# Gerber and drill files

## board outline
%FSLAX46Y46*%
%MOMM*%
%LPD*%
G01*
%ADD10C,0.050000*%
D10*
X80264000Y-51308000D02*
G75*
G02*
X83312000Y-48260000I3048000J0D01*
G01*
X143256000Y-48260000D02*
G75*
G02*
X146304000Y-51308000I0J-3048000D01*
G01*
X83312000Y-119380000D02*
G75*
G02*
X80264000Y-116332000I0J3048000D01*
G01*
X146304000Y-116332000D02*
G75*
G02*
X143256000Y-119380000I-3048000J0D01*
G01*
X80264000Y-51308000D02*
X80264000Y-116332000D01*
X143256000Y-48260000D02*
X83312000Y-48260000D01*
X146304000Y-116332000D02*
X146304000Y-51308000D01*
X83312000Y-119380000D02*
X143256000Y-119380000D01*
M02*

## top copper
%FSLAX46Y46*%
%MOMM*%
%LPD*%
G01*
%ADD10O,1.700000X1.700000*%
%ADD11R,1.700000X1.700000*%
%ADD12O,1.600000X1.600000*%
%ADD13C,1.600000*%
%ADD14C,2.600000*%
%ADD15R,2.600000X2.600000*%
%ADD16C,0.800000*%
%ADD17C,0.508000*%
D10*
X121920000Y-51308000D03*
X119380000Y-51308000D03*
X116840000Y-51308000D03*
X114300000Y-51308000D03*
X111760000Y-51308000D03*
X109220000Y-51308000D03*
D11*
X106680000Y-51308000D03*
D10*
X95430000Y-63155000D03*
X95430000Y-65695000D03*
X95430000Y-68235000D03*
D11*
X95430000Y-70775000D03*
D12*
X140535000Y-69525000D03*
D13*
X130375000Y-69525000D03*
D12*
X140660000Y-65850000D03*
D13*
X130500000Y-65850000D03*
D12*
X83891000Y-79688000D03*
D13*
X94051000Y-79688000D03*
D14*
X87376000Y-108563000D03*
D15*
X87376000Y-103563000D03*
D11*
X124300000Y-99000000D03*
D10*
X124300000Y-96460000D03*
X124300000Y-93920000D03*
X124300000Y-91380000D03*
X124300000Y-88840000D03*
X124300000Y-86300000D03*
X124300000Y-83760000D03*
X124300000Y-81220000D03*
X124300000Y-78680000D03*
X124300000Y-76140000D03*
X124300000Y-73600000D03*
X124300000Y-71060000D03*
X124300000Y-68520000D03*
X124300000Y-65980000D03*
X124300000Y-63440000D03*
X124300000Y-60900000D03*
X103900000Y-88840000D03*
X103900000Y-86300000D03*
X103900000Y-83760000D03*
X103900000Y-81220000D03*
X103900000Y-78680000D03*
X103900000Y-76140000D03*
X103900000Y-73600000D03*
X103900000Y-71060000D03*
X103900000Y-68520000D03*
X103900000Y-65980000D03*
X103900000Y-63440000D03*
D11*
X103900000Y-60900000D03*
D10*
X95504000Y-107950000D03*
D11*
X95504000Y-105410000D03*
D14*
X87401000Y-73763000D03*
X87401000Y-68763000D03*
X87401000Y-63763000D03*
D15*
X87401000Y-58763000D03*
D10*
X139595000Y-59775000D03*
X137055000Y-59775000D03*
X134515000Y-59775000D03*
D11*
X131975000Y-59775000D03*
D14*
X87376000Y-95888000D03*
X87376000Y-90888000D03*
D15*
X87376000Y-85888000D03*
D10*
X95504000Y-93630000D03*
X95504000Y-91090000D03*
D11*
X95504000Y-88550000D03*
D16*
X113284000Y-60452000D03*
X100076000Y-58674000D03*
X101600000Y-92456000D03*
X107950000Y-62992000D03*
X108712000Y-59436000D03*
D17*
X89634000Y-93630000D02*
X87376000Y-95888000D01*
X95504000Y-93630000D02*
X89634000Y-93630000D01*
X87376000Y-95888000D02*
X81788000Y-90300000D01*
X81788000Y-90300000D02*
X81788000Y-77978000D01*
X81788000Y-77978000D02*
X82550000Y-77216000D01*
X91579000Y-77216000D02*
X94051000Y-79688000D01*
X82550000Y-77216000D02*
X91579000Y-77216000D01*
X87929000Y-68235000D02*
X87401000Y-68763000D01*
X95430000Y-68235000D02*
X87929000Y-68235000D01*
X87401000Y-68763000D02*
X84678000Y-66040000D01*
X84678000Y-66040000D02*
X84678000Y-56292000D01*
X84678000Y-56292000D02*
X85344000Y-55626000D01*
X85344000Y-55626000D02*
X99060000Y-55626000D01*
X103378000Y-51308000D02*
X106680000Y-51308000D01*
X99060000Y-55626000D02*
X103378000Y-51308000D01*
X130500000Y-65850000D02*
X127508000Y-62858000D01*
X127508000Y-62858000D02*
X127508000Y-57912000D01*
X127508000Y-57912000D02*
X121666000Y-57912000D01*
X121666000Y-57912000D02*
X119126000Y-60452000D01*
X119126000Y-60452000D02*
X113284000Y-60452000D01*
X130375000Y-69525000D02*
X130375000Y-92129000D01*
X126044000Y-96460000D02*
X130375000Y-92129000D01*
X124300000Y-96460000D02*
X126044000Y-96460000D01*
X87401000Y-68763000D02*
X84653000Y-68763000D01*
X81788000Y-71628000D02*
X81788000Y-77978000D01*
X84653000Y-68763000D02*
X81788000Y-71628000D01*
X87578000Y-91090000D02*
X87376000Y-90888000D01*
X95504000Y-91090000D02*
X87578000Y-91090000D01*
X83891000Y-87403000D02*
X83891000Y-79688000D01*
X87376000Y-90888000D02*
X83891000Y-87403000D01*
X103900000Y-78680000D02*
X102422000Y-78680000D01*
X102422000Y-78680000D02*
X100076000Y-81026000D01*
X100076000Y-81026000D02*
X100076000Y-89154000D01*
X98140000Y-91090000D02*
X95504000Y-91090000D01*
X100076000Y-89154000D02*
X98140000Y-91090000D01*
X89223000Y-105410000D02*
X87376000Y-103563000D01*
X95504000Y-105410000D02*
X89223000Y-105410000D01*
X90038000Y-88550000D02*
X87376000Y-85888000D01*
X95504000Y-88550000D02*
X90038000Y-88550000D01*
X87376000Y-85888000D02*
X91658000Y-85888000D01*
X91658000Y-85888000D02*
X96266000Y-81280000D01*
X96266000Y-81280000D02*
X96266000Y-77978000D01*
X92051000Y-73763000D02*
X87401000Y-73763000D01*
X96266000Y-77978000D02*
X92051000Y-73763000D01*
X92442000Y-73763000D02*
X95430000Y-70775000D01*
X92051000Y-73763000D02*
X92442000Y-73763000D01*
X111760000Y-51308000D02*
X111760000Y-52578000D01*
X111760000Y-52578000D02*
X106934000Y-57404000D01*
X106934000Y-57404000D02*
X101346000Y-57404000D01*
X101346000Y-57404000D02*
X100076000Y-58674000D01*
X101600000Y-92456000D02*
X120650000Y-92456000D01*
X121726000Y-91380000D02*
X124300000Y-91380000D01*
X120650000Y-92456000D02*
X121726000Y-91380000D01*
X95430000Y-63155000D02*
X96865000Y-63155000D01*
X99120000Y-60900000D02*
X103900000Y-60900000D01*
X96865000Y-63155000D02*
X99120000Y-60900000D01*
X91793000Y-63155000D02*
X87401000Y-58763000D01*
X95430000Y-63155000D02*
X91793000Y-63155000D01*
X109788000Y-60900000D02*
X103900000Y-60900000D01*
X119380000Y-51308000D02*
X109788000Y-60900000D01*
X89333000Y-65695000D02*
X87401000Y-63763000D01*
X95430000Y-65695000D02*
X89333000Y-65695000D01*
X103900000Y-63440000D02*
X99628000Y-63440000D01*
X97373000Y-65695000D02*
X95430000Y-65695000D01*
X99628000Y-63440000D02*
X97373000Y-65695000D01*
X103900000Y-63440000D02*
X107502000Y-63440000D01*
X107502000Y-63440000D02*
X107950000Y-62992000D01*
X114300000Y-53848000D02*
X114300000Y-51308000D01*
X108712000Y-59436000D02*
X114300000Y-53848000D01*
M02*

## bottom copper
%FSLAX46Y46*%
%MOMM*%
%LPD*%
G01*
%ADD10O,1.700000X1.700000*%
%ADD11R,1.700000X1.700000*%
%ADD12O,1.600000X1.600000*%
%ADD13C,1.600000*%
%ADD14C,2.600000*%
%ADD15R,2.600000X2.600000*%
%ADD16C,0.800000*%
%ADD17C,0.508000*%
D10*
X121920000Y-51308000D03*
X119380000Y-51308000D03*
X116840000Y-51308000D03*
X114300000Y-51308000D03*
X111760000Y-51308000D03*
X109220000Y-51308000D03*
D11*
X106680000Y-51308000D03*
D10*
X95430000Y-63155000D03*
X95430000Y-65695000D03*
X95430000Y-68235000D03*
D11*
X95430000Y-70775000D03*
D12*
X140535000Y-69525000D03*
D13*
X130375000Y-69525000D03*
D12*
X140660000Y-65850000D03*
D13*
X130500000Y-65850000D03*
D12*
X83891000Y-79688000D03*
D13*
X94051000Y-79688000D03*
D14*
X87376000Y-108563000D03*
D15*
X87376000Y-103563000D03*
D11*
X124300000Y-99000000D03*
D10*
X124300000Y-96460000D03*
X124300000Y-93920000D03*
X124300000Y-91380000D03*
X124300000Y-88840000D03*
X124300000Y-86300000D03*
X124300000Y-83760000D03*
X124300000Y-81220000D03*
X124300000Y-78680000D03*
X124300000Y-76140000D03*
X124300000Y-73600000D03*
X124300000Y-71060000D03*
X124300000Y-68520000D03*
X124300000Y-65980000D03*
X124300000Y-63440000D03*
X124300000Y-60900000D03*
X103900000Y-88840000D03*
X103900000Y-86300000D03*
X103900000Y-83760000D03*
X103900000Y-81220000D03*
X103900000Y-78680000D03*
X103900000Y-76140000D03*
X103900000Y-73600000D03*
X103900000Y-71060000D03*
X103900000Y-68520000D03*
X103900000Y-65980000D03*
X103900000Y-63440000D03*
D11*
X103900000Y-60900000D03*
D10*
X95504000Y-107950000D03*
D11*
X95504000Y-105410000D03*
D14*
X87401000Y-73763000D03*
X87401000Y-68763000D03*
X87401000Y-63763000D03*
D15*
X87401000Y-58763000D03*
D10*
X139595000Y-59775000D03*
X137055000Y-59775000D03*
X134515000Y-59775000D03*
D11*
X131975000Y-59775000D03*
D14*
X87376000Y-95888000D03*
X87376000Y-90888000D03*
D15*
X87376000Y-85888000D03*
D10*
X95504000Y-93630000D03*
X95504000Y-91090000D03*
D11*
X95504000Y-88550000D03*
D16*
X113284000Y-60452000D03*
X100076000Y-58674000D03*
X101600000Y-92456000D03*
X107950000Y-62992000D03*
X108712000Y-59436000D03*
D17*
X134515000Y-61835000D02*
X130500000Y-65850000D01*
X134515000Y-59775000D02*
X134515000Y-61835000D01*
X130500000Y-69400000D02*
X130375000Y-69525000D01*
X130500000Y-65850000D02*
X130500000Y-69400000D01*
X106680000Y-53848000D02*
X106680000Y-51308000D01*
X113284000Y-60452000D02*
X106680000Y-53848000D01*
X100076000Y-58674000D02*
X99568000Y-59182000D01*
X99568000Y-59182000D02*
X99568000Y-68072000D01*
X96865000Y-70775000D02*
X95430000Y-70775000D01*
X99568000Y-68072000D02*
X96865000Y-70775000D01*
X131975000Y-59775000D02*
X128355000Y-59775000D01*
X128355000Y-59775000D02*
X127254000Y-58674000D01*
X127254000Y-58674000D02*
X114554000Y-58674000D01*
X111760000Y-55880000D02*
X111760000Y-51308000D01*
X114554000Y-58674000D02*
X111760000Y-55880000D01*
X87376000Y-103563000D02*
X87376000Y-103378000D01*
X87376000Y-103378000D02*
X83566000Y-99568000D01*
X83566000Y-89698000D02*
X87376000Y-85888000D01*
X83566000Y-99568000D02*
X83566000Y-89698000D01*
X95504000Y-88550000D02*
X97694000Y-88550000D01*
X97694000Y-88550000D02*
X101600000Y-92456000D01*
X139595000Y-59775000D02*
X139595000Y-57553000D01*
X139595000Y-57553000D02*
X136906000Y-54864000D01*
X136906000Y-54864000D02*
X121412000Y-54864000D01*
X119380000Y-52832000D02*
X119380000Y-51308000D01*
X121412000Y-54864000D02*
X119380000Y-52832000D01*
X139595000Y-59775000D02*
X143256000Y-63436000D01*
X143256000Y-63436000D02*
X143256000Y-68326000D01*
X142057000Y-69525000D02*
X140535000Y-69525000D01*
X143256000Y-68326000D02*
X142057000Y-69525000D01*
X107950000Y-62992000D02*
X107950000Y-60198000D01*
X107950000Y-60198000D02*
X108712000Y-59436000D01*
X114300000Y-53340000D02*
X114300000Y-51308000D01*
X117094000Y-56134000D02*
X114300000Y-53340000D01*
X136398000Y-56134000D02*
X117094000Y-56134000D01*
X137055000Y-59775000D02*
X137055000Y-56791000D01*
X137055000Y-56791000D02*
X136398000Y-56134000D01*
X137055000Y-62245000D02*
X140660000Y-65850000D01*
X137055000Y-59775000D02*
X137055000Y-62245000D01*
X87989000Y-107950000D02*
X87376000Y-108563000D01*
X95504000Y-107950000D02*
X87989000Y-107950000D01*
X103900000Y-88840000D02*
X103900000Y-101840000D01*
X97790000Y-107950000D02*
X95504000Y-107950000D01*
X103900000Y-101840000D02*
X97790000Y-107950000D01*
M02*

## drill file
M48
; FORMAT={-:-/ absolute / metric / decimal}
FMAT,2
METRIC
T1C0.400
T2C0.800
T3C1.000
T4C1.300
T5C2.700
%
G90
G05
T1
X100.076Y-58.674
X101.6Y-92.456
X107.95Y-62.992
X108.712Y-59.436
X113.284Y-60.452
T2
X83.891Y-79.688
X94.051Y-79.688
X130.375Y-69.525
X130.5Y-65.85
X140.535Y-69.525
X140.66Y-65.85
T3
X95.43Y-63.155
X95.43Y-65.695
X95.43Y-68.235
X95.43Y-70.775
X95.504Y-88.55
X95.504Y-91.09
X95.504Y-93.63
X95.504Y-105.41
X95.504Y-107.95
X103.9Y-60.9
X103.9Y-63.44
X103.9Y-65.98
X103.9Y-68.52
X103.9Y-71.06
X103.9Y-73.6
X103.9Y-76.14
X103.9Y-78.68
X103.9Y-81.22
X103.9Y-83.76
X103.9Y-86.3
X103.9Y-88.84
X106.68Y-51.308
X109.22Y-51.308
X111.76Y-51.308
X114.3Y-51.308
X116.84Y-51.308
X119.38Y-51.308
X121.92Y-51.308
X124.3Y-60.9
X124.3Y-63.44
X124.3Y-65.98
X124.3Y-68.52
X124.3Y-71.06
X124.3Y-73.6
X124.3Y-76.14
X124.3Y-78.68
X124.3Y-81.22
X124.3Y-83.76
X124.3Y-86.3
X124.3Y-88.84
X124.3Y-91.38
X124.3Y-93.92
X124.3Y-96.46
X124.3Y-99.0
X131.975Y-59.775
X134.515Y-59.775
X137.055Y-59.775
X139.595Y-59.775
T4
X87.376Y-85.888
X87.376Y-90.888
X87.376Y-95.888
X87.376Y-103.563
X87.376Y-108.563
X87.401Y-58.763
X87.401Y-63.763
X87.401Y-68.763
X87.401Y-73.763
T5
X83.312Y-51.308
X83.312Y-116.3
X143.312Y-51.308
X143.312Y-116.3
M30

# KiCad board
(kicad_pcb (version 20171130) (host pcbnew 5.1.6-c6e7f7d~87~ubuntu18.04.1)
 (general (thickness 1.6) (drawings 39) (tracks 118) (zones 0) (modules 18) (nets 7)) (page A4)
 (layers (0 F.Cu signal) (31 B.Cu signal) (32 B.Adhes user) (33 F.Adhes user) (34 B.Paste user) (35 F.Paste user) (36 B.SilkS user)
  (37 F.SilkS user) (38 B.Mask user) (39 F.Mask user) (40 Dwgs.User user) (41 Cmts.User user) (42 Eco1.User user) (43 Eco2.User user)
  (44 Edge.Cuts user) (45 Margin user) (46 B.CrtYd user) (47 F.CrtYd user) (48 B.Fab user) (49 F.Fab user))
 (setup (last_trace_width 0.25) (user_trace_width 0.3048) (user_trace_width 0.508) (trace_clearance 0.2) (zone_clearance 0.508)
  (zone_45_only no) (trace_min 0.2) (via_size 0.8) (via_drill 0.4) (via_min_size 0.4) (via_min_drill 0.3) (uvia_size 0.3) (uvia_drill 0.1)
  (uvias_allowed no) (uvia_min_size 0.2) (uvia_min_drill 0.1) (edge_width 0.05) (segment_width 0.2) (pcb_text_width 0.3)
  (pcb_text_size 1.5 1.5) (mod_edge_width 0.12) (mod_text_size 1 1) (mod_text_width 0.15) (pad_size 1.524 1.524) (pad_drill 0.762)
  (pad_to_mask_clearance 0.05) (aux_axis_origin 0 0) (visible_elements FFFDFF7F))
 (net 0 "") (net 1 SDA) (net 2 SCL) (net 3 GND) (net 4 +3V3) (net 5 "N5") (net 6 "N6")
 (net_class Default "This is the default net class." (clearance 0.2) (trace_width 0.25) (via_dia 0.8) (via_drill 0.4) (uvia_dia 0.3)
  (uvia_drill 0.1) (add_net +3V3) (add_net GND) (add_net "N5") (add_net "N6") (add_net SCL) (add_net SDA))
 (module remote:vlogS (layer F.Cu) (at 136.652 107.442)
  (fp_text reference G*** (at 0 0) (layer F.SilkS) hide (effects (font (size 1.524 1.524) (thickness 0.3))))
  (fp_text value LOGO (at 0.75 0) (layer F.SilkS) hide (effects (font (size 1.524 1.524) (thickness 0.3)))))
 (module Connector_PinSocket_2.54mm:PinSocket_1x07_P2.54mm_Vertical (layer F.Cu) (at 106.68 51.308 90)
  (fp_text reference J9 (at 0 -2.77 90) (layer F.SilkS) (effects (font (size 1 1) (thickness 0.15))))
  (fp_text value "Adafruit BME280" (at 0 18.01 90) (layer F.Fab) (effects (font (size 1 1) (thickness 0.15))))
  (pad 7 thru_hole oval (at 0 15.24 90) (size 1.7 1.7) (drill 1) (layers *.Cu *.Mask))
  (pad 6 thru_hole oval (at 0 12.7 90) (size 1.7 1.7) (drill 1) (layers *.Cu *.Mask) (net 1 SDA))
  (pad 5 thru_hole oval (at 0 10.16 90) (size 1.7 1.7) (drill 1) (layers *.Cu *.Mask))
  (pad 4 thru_hole oval (at 0 7.62 90) (size 1.7 1.7) (drill 1) (layers *.Cu *.Mask) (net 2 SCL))
  (pad 3 thru_hole oval (at 0 5.08 90) (size 1.7 1.7) (drill 1) (layers *.Cu *.Mask) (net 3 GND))
  (pad 2 thru_hole oval (at 0 2.54 90) (size 1.7 1.7) (drill 1) (layers *.Cu *.Mask))
  (pad 1 thru_hole rect (at 0 0 90) (size 1.7 1.7) (drill 1) (layers *.Cu *.Mask) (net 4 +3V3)))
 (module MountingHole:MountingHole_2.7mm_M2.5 (layer F.Cu) (at 143.312 116.3)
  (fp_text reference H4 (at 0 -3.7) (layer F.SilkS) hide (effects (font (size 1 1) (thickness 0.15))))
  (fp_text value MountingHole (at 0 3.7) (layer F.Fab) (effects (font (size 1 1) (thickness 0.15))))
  (pad 1 np_thru_hole circle (at 0 0) (size 2.7 2.7) (drill 2.7) (layers *.Cu *.Mask)))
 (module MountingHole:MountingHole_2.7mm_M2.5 (layer F.Cu) (at 83.312 116.3)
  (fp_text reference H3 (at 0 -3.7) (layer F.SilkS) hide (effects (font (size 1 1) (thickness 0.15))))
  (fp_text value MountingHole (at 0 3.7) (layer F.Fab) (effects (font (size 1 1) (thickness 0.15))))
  (pad 1 np_thru_hole circle (at 0 0) (size 2.7 2.7) (drill 2.7) (layers *.Cu *.Mask)))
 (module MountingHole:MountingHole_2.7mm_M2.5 (layer F.Cu) (at 143.312 51.308)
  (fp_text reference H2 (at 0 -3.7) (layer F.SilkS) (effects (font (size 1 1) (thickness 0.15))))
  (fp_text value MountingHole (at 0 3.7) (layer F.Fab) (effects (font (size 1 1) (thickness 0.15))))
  (pad 1 np_thru_hole circle (at 0 0) (size 2.7 2.7) (drill 2.7) (layers *.Cu *.Mask)))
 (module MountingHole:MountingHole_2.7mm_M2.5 (layer F.Cu) (at 83.312 51.308)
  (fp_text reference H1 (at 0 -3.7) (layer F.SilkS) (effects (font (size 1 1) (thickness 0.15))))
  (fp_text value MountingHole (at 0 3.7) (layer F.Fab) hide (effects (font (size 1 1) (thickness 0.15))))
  (pad 1 np_thru_hole circle (at 0 0) (size 2.7 2.7) (drill 2.7) (layers *.Cu *.Mask)))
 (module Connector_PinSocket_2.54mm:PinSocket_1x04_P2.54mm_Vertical (layer F.Cu) (at 95.43 70.775 180)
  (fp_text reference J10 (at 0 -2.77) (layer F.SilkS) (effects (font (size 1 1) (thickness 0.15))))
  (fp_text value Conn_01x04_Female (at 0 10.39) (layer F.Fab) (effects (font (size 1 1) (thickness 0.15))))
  (pad 4 thru_hole oval (at 0 7.62 180) (size 1.7 1.7) (drill 1) (layers *.Cu *.Mask) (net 1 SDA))
  (pad 3 thru_hole oval (at 0 5.08 180) (size 1.7 1.7) (drill 1) (layers *.Cu *.Mask) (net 2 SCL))
  (pad 2 thru_hole oval (at 0 2.54 180) (size 1.7 1.7) (drill 1) (layers *.Cu *.Mask) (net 4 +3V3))
  (pad 1 thru_hole rect (at 0 0 180) (size 1.7 1.7) (drill 1) (layers *.Cu *.Mask) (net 3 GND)))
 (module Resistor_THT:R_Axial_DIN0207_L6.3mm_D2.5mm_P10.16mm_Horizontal (layer F.Cu) (at 130.375 69.525)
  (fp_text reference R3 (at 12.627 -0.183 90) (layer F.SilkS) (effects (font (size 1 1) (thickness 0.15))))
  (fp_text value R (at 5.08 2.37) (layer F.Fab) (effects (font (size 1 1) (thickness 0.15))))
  (pad 2 thru_hole oval (at 10.16 0) (size 1.6 1.6) (drill 0.8) (layers *.Cu *.Mask) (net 1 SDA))
  (pad 1 thru_hole circle (at 0 0) (size 1.6 1.6) (drill 0.8) (layers *.Cu *.Mask) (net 4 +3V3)))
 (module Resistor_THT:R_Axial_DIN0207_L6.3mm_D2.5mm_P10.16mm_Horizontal (layer F.Cu) (at 130.5 65.85)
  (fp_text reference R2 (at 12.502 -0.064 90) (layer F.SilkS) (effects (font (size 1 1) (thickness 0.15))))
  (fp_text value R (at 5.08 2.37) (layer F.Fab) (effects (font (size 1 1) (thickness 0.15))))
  (pad 2 thru_hole oval (at 10.16 0) (size 1.6 1.6) (drill 0.8) (layers *.Cu *.Mask) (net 2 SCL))
  (pad 1 thru_hole circle (at 0 0) (size 1.6 1.6) (drill 0.8) (layers *.Cu *.Mask) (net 4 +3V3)))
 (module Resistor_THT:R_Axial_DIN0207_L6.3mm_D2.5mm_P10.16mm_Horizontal (layer F.Cu) (at 94.051 79.688 180)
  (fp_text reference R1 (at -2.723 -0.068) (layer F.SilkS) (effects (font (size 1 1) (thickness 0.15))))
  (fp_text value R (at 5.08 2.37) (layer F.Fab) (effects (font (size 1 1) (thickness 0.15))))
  (pad 2 thru_hole oval (at 10.16 0 180) (size 1.6 1.6) (drill 0.8) (layers *.Cu *.Mask) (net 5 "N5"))
  (pad 1 thru_hole circle (at 0 0 180) (size 1.6 1.6) (drill 0.8) (layers *.Cu *.Mask) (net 4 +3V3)))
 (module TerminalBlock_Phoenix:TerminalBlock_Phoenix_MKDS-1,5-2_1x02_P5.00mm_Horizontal (layer F.Cu) (at 87.376 103.563 270)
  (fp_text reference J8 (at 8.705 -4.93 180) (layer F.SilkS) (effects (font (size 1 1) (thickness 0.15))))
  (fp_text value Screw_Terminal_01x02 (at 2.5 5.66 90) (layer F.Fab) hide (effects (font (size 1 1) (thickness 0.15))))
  (pad 2 thru_hole circle (at 5 0 270) (size 2.6 2.6) (drill 1.3) (layers *.Cu *.Mask) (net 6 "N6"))
  (pad 1 thru_hole rect (at 0 0 270) (size 2.6 2.6) (drill 1.3) (layers *.Cu *.Mask) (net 3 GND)))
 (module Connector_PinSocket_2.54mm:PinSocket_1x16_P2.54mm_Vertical (layer F.Cu) (at 124.3 99 180)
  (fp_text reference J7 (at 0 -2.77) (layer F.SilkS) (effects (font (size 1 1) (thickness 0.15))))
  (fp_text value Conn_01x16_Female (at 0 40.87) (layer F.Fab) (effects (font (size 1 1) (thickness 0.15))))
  (pad 1 thru_hole rect (at 0 0 180) (size 1.7 1.7) (drill 1) (layers *.Cu *.Mask))
  (pad 2 thru_hole oval (at 0 2.54 180) (size 1.7 1.7) (drill 1) (layers *.Cu *.Mask) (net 4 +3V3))
  (pad 3 thru_hole oval (at 0 5.08 180) (size 1.7 1.7) (drill 1) (layers *.Cu *.Mask))
  (pad 4 thru_hole oval (at 0 7.62 180) (size 1.7 1.7) (drill 1) (layers *.Cu *.Mask) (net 3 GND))
  (pad 5 thru_hole oval (at 0 10.16 180) (size 1.7 1.7) (drill 1) (layers *.Cu *.Mask))
  (pad 6 thru_hole oval (at 0 12.7 180) (size 1.7 1.7) (drill 1) (layers *.Cu *.Mask))
  (pad 7 thru_hole oval (at 0 15.24 180) (size 1.7 1.7) (drill 1) (layers *.Cu *.Mask))
  (pad 8 thru_hole oval (at 0 17.78 180) (size 1.7 1.7) (drill 1) (layers *.Cu *.Mask))
  (pad 9 thru_hole oval (at 0 20.32 180) (size 1.7 1.7) (drill 1) (layers *.Cu *.Mask))
  (pad 10 thru_hole oval (at 0 22.86 180) (size 1.7 1.7) (drill 1) (layers *.Cu *.Mask))
  (pad 11 thru_hole oval (at 0 25.4 180) (size 1.7 1.7) (drill 1) (layers *.Cu *.Mask))
  (pad 12 thru_hole oval (at 0 27.94 180) (size 1.7 1.7) (drill 1) (layers *.Cu *.Mask))
  (pad 13 thru_hole oval (at 0 30.48 180) (size 1.7 1.7) (drill 1) (layers *.Cu *.Mask))
  (pad 14 thru_hole oval (at 0 33.02 180) (size 1.7 1.7) (drill 1) (layers *.Cu *.Mask))
  (pad 15 thru_hole oval (at 0 35.56 180) (size 1.7 1.7) (drill 1) (layers *.Cu *.Mask))
  (pad 16 thru_hole oval (at 0 38.1 180) (size 1.7 1.7) (drill 1) (layers *.Cu *.Mask)))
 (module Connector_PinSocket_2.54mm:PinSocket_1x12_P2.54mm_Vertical (layer F.Cu) (at 103.9 60.9)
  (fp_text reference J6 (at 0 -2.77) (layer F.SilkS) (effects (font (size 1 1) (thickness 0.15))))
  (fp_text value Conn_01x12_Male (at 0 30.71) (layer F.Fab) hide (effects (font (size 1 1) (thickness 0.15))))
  (pad 12 thru_hole oval (at 0 27.94) (size 1.7 1.7) (drill 1) (layers *.Cu *.Mask) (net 6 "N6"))
  (pad 11 thru_hole oval (at 0 25.4) (size 1.7 1.7) (drill 1) (layers *.Cu *.Mask))
  (pad 10 thru_hole oval (at 0 22.86) (size 1.7 1.7) (drill 1) (layers *.Cu *.Mask))
  (pad 9 thru_hole oval (at 0 20.32) (size 1.7 1.7) (drill 1) (layers *.Cu *.Mask))
  (pad 8 thru_hole oval (at 0 17.78) (size 1.7 1.7) (drill 1) (layers *.Cu *.Mask) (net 5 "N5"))
  (pad 7 thru_hole oval (at 0 15.24) (size 1.7 1.7) (drill 1) (layers *.Cu *.Mask))
  (pad 6 thru_hole oval (at 0 12.7) (size 1.7 1.7) (drill 1) (layers *.Cu *.Mask))
  (pad 5 thru_hole oval (at 0 10.16) (size 1.7 1.7) (drill 1) (layers *.Cu *.Mask))
  (pad 4 thru_hole oval (at 0 7.62) (size 1.7 1.7) (drill 1) (layers *.Cu *.Mask))
  (pad 3 thru_hole oval (at 0 5.08) (size 1.7 1.7) (drill 1) (layers *.Cu *.Mask))
  (pad 2 thru_hole oval (at 0 2.54) (size 1.7 1.7) (drill 1) (layers *.Cu *.Mask) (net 2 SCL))
  (pad 1 thru_hole rect (at 0 0) (size 1.7 1.7) (drill 1) (layers *.Cu *.Mask) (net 1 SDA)))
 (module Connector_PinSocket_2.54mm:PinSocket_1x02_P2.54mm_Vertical (layer F.Cu) (at 95.504 105.41)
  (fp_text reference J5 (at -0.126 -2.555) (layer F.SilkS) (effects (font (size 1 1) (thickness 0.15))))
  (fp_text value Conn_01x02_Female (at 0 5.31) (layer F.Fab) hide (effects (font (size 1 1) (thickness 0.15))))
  (pad 2 thru_hole oval (at 0 2.54) (size 1.7 1.7) (drill 1) (layers *.Cu *.Mask) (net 6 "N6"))
  (pad 1 thru_hole rect (at 0 0) (size 1.7 1.7) (drill 1) (layers *.Cu *.Mask) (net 3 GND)))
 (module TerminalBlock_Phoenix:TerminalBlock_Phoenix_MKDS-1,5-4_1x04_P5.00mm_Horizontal (layer F.Cu) (at 87.401 58.763 270)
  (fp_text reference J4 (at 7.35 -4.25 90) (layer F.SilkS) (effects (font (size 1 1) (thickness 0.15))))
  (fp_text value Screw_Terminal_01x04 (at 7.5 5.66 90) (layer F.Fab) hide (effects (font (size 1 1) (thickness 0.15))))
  (pad 4 thru_hole circle (at 15 0 270) (size 2.6 2.6) (drill 1.3) (layers *.Cu *.Mask) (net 3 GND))
  (pad 3 thru_hole circle (at 10 0 270) (size 2.6 2.6) (drill 1.3) (layers *.Cu *.Mask) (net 4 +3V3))
  (pad 2 thru_hole circle (at 5 0 270) (size 2.6 2.6) (drill 1.3) (layers *.Cu *.Mask) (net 2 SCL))
  (pad 1 thru_hole rect (at 0 0 270) (size 2.6 2.6) (drill 1.3) (layers *.Cu *.Mask) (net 1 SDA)))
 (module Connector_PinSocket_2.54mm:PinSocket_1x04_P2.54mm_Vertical (layer F.Cu) (at 131.975 59.775 90)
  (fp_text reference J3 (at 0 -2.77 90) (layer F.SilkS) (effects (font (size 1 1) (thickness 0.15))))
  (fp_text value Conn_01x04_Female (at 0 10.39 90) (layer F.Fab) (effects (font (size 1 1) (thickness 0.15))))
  (pad 4 thru_hole oval (at 0 7.62 90) (size 1.7 1.7) (drill 1) (layers *.Cu *.Mask) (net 1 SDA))
  (pad 3 thru_hole oval (at 0 5.08 90) (size 1.7 1.7) (drill 1) (layers *.Cu *.Mask) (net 2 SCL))
  (pad 2 thru_hole oval (at 0 2.54 90) (size 1.7 1.7) (drill 1) (layers *.Cu *.Mask) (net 4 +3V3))
  (pad 1 thru_hole rect (at 0 0 90) (size 1.7 1.7) (drill 1) (layers *.Cu *.Mask) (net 3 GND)))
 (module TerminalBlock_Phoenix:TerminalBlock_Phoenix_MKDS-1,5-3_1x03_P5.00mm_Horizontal (layer F.Cu) (at 87.376 85.888 270)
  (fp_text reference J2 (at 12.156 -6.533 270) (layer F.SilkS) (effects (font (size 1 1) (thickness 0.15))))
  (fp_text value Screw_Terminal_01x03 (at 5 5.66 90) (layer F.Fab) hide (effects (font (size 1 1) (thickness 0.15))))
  (pad 3 thru_hole circle (at 10 0 270) (size 2.6 2.6) (drill 1.3) (layers *.Cu *.Mask) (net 4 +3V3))
  (pad 2 thru_hole circle (at 5 0 270) (size 2.6 2.6) (drill 1.3) (layers *.Cu *.Mask) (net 5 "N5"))
  (pad 1 thru_hole rect (at 0 0 270) (size 2.6 2.6) (drill 1.3) (layers *.Cu *.Mask) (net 3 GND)))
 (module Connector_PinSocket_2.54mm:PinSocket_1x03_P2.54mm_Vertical (layer F.Cu) (at 95.504 88.55)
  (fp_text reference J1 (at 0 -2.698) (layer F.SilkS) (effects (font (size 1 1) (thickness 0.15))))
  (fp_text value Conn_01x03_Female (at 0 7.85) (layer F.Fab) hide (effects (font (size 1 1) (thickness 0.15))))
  (pad 3 thru_hole oval (at 0 5.08) (size 1.7 1.7) (drill 1) (layers *.Cu *.Mask) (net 4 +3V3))
  (pad 2 thru_hole oval (at 0 2.54) (size 1.7 1.7) (drill 1) (layers *.Cu *.Mask) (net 5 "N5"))
  (pad 1 thru_hole rect (at 0 0) (size 1.7 1.7) (drill 1) (layers *.Cu *.Mask) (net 3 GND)))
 (gr_arc (start 83.312 51.308) (end 83.312 48.26) (angle -90) (layer Edge.Cuts) (width 0.05))
 (gr_arc (start 143.256 51.308) (end 146.304 51.308) (angle -90) (layer Edge.Cuts) (width 0.05))
 (gr_arc (start 83.312 116.332) (end 80.264 116.332) (angle -90) (layer Edge.Cuts) (width 0.05))
 (gr_arc (start 143.256 116.332) (end 143.256 119.38) (angle -90) (layer Edge.Cuts) (width 0.05))
 (gr_line (start 80.264 51.308) (end 80.264 116.332) (layer Edge.Cuts) (width 0.05))
 (gr_line (start 143.256 48.26) (end 83.312 48.26) (layer Edge.Cuts) (width 0.05))
 (gr_line (start 146.304 116.332) (end 146.304 51.308) (layer Edge.Cuts) (width 0.05))
 (gr_line (start 83.312 119.38) (end 143.256 119.38) (layer Edge.Cuts) (width 0.05))
 (segment (start 89.634 93.63) (end 87.376 95.888) (width 0.508) (layer F.Cu) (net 4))
 (segment (start 95.504 93.63) (end 89.634 93.63) (width 0.508) (layer F.Cu) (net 4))
 (segment (start 87.376 95.888) (end 81.788 90.3) (width 0.508) (layer F.Cu) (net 4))
 (segment (start 81.788 90.3) (end 81.788 77.978) (width 0.508) (layer F.Cu) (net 4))
 (segment (start 81.788 77.978) (end 82.55 77.216) (width 0.508) (layer F.Cu) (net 4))
 (segment (start 91.579 77.216) (end 94.051 79.688) (width 0.508) (layer F.Cu) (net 4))
 (segment (start 82.55 77.216) (end 91.579 77.216) (width 0.508) (layer F.Cu) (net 4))
 (segment (start 87.929 68.235) (end 87.401 68.763) (width 0.508) (layer F.Cu) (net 4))
 (segment (start 95.43 68.235) (end 87.929 68.235) (width 0.508) (layer F.Cu) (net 4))
 (segment (start 87.401 68.763) (end 84.678 66.04) (width 0.508) (layer F.Cu) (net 4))
 (segment (start 84.678 66.04) (end 84.678 56.292) (width 0.508) (layer F.Cu) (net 4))
 (segment (start 84.678 56.292) (end 85.344 55.626) (width 0.508) (layer F.Cu) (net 4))
 (segment (start 85.344 55.626) (end 99.06 55.626) (width 0.508) (layer F.Cu) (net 4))
 (segment (start 103.378 51.308) (end 106.68 51.308) (width 0.508) (layer F.Cu) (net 4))
 (segment (start 99.06 55.626) (end 103.378 51.308) (width 0.508) (layer F.Cu) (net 4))
 (segment (start 134.515 61.835) (end 130.5 65.85) (width 0.508) (layer B.Cu) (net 4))
 (segment (start 134.515 59.775) (end 134.515 61.835) (width 0.508) (layer B.Cu) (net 4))
 (segment (start 130.5 69.4) (end 130.375 69.525) (width 0.508) (layer B.Cu) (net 4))
 (segment (start 130.5 65.85) (end 130.5 69.4) (width 0.508) (layer B.Cu) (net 4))
 (segment (start 130.5 65.85) (end 127.508 62.858) (width 0.508) (layer F.Cu) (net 4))
 (segment (start 127.508 62.858) (end 127.508 57.912) (width 0.508) (layer F.Cu) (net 4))
 (segment (start 127.508 57.912) (end 121.666 57.912) (width 0.508) (layer F.Cu) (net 4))
 (via (at 113.284 60.452) (size 0.8) (drill 0.4) (layers F.Cu B.Cu) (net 4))
 (segment (start 121.666 57.912) (end 119.126 60.452) (width 0.508) (layer F.Cu) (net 4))
 (segment (start 119.126 60.452) (end 113.284 60.452) (width 0.508) (layer F.Cu) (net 4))
 (segment (start 106.68 53.848) (end 106.68 51.308) (width 0.508) (layer B.Cu) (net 4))
 (segment (start 113.284 60.452) (end 106.68 53.848) (width 0.508) (layer B.Cu) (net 4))
 (segment (start 130.375 69.525) (end 130.375 92.129) (width 0.508) (layer F.Cu) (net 4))
 (segment (start 126.044 96.46) (end 130.375 92.129) (width 0.508) (layer F.Cu) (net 4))
 (segment (start 124.3 96.46) (end 126.044 96.46) (width 0.508) (layer F.Cu) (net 4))
 (segment (start 87.401 68.763) (end 84.653 68.763) (width 0.508) (layer F.Cu) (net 4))
 (segment (start 81.788 71.628) (end 81.788 77.978) (width 0.508) (layer F.Cu) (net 4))
 (segment (start 84.653 68.763) (end 81.788 71.628) (width 0.508) (layer F.Cu) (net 4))
 (segment (start 87.578 91.09) (end 87.376 90.888) (width 0.508) (layer F.Cu) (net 5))
 (segment (start 95.504 91.09) (end 87.578 91.09) (width 0.508) (layer F.Cu) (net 5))
 (segment (start 83.891 87.403) (end 83.891 79.688) (width 0.508) (layer F.Cu) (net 5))
 (segment (start 87.376 90.888) (end 83.891 87.403) (width 0.508) (layer F.Cu) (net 5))
 (segment (start 103.9 78.68) (end 102.422 78.68) (width 0.508) (layer F.Cu) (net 5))
 (segment (start 102.422 78.68) (end 100.076 81.026) (width 0.508) (layer F.Cu) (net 5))
 (segment (start 100.076 81.026) (end 100.076 89.154) (width 0.508) (layer F.Cu) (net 5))
 (segment (start 98.14 91.09) (end 95.504 91.09) (width 0.508) (layer F.Cu) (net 5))
 (segment (start 100.076 89.154) (end 98.14 91.09) (width 0.508) (layer F.Cu) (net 5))
 (segment (start 89.223 105.41) (end 87.376 103.563) (width 0.508) (layer F.Cu) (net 3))
 (segment (start 95.504 105.41) (end 89.223 105.41) (width 0.508) (layer F.Cu) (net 3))
 (segment (start 90.038 88.55) (end 87.376 85.888) (width 0.508) (layer F.Cu) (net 3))
 (segment (start 95.504 88.55) (end 90.038 88.55) (width 0.508) (layer F.Cu) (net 3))
 (segment (start 87.376 85.888) (end 91.658 85.888) (width 0.508) (layer F.Cu) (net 3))
 (segment (start 91.658 85.888) (end 96.266 81.28) (width 0.508) (layer F.Cu) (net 3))
 (segment (start 96.266 81.28) (end 96.266 77.978) (width 0.508) (layer F.Cu) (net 3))
 (segment (start 92.051 73.763) (end 87.401 73.763) (width 0.508) (layer F.Cu) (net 3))
 (segment (start 96.266 77.978) (end 92.051 73.763) (width 0.508) (layer F.Cu) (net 3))
 (segment (start 92.442 73.763) (end 95.43 70.775) (width 0.508) (layer F.Cu) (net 3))
 (segment (start 92.051 73.763) (end 92.442 73.763) (width 0.508) (layer F.Cu) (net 3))
 (segment (start 111.76 51.308) (end 111.76 52.578) (width 0.508) (layer F.Cu) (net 3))
 (segment (start 111.76 52.578) (end 106.934 57.404) (width 0.508) (layer F.Cu) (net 3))
 (via (at 100.076 58.674) (size 0.8) (drill 0.4) (layers F.Cu B.Cu) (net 3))
 (segment (start 106.934 57.404) (end 101.346 57.404) (width 0.508) (layer F.Cu) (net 3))
 (segment (start 101.346 57.404) (end 100.076 58.674) (width 0.508) (layer F.Cu) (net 3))
 (segment (start 100.076 58.674) (end 99.568 59.182) (width 0.508) (layer B.Cu) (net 3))
 (segment (start 99.568 59.182) (end 99.568 68.072) (width 0.508) (layer B.Cu) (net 3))
 (segment (start 96.865 70.775) (end 95.43 70.775) (width 0.508) (layer B.Cu) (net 3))
 (segment (start 99.568 68.072) (end 96.865 70.775) (width 0.508) (layer B.Cu) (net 3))
 (segment (start 131.975 59.775) (end 128.355 59.775) (width 0.508) (layer B.Cu) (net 3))
 (segment (start 128.355 59.775) (end 127.254 58.674) (width 0.508) (layer B.Cu) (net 3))
 (segment (start 127.254 58.674) (end 114.554 58.674) (width 0.508) (layer B.Cu) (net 3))
 (segment (start 111.76 55.88) (end 111.76 51.308) (width 0.508) (layer B.Cu) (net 3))
 (segment (start 114.554 58.674) (end 111.76 55.88) (width 0.508) (layer B.Cu) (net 3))
 (segment (start 87.376 103.563) (end 87.376 103.378) (width 0.508) (layer B.Cu) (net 3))
 (segment (start 87.376 103.378) (end 83.566 99.568) (width 0.508) (layer B.Cu) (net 3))
 (segment (start 83.566 89.698) (end 87.376 85.888) (width 0.508) (layer B.Cu) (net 3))
 (segment (start 83.566 99.568) (end 83.566 89.698) (width 0.508) (layer B.Cu) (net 3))
 (segment (start 95.504 88.55) (end 97.694 88.55) (width 0.508) (layer B.Cu) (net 3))
 (segment (start 97.694 88.55) (end 101.6 92.456) (width 0.508) (layer B.Cu) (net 3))
 (via (at 101.6 92.456) (size 0.8) (drill 0.4) (layers F.Cu B.Cu) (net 3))
 (segment (start 101.6 92.456) (end 120.65 92.456) (width 0.508) (layer F.Cu) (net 3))
 (segment (start 121.726 91.38) (end 124.3 91.38) (width 0.508) (layer F.Cu) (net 3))
 (segment (start 120.65 92.456) (end 121.726 91.38) (width 0.508) (layer F.Cu) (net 3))
 (segment (start 95.43 63.155) (end 96.865 63.155) (width 0.508) (layer F.Cu) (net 1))
 (segment (start 99.12 60.9) (end 103.9 60.9) (width 0.508) (layer F.Cu) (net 1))
 (segment (start 96.865 63.155) (end 99.12 60.9) (width 0.508) (layer F.Cu) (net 1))
 (segment (start 91.793 63.155) (end 87.401 58.763) (width 0.508) (layer F.Cu) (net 1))
 (segment (start 95.43 63.155) (end 91.793 63.155) (width 0.508) (layer F.Cu) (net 1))
 (segment (start 109.788 60.9) (end 103.9 60.9) (width 0.508) (layer F.Cu) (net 1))
 (segment (start 119.38 51.308) (end 109.788 60.9) (width 0.508) (layer F.Cu) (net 1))
 (segment (start 139.595 59.775) (end 139.595 57.553) (width 0.508) (layer B.Cu) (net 1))
 (segment (start 139.595 57.553) (end 136.906 54.864) (width 0.508) (layer B.Cu) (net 1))
 (segment (start 136.906 54.864) (end 121.412 54.864) (width 0.508) (layer B.Cu) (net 1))
 (segment (start 119.38 52.832) (end 119.38 51.308) (width 0.508) (layer B.Cu) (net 1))
 (segment (start 121.412 54.864) (end 119.38 52.832) (width 0.508) (layer B.Cu) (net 1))
 (segment (start 139.595 59.775) (end 143.256 63.436) (width 0.508) (layer B.Cu) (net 1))
 (segment (start 143.256 63.436) (end 143.256 68.326) (width 0.508) (layer B.Cu) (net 1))
 (segment (start 142.057 69.525) (end 140.535 69.525) (width 0.508) (layer B.Cu) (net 1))
 (segment (start 143.256 68.326) (end 142.057 69.525) (width 0.508) (layer B.Cu) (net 1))
 (segment (start 89.333 65.695) (end 87.401 63.763) (width 0.508) (layer F.Cu) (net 2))
 (segment (start 95.43 65.695) (end 89.333 65.695) (width 0.508) (layer F.Cu) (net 2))
 (segment (start 103.9 63.44) (end 99.628 63.44) (width 0.508) (layer F.Cu) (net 2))
 (segment (start 97.373 65.695) (end 95.43 65.695) (width 0.508) (layer F.Cu) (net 2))
 (segment (start 99.628 63.44) (end 97.373 65.695) (width 0.508) (layer F.Cu) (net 2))
 (via (at 107.95 62.992) (size 0.8) (drill 0.4) (layers F.Cu B.Cu) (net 2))
 (segment (start 103.9 63.44) (end 107.502 63.44) (width 0.508) (layer F.Cu) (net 2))
 (segment (start 107.502 63.44) (end 107.95 62.992) (width 0.508) (layer F.Cu) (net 2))
 (via (at 108.712 59.436) (size 0.8) (drill 0.4) (layers F.Cu B.Cu) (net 2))
 (segment (start 107.95 62.992) (end 107.95 60.198) (width 0.508) (layer B.Cu) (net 2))
 (segment (start 107.95 60.198) (end 108.712 59.436) (width 0.508) (layer B.Cu) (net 2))
 (segment (start 114.3 53.848) (end 114.3 51.308) (width 0.508) (layer F.Cu) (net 2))
 (segment (start 108.712 59.436) (end 114.3 53.848) (width 0.508) (layer F.Cu) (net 2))
 (segment (start 114.3 53.34) (end 114.3 51.308) (width 0.508) (layer B.Cu) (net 2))
 (segment (start 117.094 56.134) (end 114.3 53.34) (width 0.508) (layer B.Cu) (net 2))
 (segment (start 136.398 56.134) (end 117.094 56.134) (width 0.508) (layer B.Cu) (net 2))
 (segment (start 137.055 59.775) (end 137.055 56.791) (width 0.508) (layer B.Cu) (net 2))
 (segment (start 137.055 56.791) (end 136.398 56.134) (width 0.508) (layer B.Cu) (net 2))
 (segment (start 137.055 62.245) (end 140.66 65.85) (width 0.508) (layer B.Cu) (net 2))
 (segment (start 137.055 59.775) (end 137.055 62.245) (width 0.508) (layer B.Cu) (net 2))
 (segment (start 87.989 107.95) (end 87.376 108.563) (width 0.508) (layer B.Cu) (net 6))
 (segment (start 95.504 107.95) (end 87.989 107.95) (width 0.508) (layer B.Cu) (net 6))
 (segment (start 103.9 88.84) (end 103.9 101.84) (width 0.508) (layer B.Cu) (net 6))
 (segment (start 97.79 107.95) (end 95.504 107.95) (width 0.508) (layer B.Cu) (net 6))
 (segment (start 103.9 101.84) (end 97.79 107.95) (width 0.508) (layer B.Cu) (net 6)))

